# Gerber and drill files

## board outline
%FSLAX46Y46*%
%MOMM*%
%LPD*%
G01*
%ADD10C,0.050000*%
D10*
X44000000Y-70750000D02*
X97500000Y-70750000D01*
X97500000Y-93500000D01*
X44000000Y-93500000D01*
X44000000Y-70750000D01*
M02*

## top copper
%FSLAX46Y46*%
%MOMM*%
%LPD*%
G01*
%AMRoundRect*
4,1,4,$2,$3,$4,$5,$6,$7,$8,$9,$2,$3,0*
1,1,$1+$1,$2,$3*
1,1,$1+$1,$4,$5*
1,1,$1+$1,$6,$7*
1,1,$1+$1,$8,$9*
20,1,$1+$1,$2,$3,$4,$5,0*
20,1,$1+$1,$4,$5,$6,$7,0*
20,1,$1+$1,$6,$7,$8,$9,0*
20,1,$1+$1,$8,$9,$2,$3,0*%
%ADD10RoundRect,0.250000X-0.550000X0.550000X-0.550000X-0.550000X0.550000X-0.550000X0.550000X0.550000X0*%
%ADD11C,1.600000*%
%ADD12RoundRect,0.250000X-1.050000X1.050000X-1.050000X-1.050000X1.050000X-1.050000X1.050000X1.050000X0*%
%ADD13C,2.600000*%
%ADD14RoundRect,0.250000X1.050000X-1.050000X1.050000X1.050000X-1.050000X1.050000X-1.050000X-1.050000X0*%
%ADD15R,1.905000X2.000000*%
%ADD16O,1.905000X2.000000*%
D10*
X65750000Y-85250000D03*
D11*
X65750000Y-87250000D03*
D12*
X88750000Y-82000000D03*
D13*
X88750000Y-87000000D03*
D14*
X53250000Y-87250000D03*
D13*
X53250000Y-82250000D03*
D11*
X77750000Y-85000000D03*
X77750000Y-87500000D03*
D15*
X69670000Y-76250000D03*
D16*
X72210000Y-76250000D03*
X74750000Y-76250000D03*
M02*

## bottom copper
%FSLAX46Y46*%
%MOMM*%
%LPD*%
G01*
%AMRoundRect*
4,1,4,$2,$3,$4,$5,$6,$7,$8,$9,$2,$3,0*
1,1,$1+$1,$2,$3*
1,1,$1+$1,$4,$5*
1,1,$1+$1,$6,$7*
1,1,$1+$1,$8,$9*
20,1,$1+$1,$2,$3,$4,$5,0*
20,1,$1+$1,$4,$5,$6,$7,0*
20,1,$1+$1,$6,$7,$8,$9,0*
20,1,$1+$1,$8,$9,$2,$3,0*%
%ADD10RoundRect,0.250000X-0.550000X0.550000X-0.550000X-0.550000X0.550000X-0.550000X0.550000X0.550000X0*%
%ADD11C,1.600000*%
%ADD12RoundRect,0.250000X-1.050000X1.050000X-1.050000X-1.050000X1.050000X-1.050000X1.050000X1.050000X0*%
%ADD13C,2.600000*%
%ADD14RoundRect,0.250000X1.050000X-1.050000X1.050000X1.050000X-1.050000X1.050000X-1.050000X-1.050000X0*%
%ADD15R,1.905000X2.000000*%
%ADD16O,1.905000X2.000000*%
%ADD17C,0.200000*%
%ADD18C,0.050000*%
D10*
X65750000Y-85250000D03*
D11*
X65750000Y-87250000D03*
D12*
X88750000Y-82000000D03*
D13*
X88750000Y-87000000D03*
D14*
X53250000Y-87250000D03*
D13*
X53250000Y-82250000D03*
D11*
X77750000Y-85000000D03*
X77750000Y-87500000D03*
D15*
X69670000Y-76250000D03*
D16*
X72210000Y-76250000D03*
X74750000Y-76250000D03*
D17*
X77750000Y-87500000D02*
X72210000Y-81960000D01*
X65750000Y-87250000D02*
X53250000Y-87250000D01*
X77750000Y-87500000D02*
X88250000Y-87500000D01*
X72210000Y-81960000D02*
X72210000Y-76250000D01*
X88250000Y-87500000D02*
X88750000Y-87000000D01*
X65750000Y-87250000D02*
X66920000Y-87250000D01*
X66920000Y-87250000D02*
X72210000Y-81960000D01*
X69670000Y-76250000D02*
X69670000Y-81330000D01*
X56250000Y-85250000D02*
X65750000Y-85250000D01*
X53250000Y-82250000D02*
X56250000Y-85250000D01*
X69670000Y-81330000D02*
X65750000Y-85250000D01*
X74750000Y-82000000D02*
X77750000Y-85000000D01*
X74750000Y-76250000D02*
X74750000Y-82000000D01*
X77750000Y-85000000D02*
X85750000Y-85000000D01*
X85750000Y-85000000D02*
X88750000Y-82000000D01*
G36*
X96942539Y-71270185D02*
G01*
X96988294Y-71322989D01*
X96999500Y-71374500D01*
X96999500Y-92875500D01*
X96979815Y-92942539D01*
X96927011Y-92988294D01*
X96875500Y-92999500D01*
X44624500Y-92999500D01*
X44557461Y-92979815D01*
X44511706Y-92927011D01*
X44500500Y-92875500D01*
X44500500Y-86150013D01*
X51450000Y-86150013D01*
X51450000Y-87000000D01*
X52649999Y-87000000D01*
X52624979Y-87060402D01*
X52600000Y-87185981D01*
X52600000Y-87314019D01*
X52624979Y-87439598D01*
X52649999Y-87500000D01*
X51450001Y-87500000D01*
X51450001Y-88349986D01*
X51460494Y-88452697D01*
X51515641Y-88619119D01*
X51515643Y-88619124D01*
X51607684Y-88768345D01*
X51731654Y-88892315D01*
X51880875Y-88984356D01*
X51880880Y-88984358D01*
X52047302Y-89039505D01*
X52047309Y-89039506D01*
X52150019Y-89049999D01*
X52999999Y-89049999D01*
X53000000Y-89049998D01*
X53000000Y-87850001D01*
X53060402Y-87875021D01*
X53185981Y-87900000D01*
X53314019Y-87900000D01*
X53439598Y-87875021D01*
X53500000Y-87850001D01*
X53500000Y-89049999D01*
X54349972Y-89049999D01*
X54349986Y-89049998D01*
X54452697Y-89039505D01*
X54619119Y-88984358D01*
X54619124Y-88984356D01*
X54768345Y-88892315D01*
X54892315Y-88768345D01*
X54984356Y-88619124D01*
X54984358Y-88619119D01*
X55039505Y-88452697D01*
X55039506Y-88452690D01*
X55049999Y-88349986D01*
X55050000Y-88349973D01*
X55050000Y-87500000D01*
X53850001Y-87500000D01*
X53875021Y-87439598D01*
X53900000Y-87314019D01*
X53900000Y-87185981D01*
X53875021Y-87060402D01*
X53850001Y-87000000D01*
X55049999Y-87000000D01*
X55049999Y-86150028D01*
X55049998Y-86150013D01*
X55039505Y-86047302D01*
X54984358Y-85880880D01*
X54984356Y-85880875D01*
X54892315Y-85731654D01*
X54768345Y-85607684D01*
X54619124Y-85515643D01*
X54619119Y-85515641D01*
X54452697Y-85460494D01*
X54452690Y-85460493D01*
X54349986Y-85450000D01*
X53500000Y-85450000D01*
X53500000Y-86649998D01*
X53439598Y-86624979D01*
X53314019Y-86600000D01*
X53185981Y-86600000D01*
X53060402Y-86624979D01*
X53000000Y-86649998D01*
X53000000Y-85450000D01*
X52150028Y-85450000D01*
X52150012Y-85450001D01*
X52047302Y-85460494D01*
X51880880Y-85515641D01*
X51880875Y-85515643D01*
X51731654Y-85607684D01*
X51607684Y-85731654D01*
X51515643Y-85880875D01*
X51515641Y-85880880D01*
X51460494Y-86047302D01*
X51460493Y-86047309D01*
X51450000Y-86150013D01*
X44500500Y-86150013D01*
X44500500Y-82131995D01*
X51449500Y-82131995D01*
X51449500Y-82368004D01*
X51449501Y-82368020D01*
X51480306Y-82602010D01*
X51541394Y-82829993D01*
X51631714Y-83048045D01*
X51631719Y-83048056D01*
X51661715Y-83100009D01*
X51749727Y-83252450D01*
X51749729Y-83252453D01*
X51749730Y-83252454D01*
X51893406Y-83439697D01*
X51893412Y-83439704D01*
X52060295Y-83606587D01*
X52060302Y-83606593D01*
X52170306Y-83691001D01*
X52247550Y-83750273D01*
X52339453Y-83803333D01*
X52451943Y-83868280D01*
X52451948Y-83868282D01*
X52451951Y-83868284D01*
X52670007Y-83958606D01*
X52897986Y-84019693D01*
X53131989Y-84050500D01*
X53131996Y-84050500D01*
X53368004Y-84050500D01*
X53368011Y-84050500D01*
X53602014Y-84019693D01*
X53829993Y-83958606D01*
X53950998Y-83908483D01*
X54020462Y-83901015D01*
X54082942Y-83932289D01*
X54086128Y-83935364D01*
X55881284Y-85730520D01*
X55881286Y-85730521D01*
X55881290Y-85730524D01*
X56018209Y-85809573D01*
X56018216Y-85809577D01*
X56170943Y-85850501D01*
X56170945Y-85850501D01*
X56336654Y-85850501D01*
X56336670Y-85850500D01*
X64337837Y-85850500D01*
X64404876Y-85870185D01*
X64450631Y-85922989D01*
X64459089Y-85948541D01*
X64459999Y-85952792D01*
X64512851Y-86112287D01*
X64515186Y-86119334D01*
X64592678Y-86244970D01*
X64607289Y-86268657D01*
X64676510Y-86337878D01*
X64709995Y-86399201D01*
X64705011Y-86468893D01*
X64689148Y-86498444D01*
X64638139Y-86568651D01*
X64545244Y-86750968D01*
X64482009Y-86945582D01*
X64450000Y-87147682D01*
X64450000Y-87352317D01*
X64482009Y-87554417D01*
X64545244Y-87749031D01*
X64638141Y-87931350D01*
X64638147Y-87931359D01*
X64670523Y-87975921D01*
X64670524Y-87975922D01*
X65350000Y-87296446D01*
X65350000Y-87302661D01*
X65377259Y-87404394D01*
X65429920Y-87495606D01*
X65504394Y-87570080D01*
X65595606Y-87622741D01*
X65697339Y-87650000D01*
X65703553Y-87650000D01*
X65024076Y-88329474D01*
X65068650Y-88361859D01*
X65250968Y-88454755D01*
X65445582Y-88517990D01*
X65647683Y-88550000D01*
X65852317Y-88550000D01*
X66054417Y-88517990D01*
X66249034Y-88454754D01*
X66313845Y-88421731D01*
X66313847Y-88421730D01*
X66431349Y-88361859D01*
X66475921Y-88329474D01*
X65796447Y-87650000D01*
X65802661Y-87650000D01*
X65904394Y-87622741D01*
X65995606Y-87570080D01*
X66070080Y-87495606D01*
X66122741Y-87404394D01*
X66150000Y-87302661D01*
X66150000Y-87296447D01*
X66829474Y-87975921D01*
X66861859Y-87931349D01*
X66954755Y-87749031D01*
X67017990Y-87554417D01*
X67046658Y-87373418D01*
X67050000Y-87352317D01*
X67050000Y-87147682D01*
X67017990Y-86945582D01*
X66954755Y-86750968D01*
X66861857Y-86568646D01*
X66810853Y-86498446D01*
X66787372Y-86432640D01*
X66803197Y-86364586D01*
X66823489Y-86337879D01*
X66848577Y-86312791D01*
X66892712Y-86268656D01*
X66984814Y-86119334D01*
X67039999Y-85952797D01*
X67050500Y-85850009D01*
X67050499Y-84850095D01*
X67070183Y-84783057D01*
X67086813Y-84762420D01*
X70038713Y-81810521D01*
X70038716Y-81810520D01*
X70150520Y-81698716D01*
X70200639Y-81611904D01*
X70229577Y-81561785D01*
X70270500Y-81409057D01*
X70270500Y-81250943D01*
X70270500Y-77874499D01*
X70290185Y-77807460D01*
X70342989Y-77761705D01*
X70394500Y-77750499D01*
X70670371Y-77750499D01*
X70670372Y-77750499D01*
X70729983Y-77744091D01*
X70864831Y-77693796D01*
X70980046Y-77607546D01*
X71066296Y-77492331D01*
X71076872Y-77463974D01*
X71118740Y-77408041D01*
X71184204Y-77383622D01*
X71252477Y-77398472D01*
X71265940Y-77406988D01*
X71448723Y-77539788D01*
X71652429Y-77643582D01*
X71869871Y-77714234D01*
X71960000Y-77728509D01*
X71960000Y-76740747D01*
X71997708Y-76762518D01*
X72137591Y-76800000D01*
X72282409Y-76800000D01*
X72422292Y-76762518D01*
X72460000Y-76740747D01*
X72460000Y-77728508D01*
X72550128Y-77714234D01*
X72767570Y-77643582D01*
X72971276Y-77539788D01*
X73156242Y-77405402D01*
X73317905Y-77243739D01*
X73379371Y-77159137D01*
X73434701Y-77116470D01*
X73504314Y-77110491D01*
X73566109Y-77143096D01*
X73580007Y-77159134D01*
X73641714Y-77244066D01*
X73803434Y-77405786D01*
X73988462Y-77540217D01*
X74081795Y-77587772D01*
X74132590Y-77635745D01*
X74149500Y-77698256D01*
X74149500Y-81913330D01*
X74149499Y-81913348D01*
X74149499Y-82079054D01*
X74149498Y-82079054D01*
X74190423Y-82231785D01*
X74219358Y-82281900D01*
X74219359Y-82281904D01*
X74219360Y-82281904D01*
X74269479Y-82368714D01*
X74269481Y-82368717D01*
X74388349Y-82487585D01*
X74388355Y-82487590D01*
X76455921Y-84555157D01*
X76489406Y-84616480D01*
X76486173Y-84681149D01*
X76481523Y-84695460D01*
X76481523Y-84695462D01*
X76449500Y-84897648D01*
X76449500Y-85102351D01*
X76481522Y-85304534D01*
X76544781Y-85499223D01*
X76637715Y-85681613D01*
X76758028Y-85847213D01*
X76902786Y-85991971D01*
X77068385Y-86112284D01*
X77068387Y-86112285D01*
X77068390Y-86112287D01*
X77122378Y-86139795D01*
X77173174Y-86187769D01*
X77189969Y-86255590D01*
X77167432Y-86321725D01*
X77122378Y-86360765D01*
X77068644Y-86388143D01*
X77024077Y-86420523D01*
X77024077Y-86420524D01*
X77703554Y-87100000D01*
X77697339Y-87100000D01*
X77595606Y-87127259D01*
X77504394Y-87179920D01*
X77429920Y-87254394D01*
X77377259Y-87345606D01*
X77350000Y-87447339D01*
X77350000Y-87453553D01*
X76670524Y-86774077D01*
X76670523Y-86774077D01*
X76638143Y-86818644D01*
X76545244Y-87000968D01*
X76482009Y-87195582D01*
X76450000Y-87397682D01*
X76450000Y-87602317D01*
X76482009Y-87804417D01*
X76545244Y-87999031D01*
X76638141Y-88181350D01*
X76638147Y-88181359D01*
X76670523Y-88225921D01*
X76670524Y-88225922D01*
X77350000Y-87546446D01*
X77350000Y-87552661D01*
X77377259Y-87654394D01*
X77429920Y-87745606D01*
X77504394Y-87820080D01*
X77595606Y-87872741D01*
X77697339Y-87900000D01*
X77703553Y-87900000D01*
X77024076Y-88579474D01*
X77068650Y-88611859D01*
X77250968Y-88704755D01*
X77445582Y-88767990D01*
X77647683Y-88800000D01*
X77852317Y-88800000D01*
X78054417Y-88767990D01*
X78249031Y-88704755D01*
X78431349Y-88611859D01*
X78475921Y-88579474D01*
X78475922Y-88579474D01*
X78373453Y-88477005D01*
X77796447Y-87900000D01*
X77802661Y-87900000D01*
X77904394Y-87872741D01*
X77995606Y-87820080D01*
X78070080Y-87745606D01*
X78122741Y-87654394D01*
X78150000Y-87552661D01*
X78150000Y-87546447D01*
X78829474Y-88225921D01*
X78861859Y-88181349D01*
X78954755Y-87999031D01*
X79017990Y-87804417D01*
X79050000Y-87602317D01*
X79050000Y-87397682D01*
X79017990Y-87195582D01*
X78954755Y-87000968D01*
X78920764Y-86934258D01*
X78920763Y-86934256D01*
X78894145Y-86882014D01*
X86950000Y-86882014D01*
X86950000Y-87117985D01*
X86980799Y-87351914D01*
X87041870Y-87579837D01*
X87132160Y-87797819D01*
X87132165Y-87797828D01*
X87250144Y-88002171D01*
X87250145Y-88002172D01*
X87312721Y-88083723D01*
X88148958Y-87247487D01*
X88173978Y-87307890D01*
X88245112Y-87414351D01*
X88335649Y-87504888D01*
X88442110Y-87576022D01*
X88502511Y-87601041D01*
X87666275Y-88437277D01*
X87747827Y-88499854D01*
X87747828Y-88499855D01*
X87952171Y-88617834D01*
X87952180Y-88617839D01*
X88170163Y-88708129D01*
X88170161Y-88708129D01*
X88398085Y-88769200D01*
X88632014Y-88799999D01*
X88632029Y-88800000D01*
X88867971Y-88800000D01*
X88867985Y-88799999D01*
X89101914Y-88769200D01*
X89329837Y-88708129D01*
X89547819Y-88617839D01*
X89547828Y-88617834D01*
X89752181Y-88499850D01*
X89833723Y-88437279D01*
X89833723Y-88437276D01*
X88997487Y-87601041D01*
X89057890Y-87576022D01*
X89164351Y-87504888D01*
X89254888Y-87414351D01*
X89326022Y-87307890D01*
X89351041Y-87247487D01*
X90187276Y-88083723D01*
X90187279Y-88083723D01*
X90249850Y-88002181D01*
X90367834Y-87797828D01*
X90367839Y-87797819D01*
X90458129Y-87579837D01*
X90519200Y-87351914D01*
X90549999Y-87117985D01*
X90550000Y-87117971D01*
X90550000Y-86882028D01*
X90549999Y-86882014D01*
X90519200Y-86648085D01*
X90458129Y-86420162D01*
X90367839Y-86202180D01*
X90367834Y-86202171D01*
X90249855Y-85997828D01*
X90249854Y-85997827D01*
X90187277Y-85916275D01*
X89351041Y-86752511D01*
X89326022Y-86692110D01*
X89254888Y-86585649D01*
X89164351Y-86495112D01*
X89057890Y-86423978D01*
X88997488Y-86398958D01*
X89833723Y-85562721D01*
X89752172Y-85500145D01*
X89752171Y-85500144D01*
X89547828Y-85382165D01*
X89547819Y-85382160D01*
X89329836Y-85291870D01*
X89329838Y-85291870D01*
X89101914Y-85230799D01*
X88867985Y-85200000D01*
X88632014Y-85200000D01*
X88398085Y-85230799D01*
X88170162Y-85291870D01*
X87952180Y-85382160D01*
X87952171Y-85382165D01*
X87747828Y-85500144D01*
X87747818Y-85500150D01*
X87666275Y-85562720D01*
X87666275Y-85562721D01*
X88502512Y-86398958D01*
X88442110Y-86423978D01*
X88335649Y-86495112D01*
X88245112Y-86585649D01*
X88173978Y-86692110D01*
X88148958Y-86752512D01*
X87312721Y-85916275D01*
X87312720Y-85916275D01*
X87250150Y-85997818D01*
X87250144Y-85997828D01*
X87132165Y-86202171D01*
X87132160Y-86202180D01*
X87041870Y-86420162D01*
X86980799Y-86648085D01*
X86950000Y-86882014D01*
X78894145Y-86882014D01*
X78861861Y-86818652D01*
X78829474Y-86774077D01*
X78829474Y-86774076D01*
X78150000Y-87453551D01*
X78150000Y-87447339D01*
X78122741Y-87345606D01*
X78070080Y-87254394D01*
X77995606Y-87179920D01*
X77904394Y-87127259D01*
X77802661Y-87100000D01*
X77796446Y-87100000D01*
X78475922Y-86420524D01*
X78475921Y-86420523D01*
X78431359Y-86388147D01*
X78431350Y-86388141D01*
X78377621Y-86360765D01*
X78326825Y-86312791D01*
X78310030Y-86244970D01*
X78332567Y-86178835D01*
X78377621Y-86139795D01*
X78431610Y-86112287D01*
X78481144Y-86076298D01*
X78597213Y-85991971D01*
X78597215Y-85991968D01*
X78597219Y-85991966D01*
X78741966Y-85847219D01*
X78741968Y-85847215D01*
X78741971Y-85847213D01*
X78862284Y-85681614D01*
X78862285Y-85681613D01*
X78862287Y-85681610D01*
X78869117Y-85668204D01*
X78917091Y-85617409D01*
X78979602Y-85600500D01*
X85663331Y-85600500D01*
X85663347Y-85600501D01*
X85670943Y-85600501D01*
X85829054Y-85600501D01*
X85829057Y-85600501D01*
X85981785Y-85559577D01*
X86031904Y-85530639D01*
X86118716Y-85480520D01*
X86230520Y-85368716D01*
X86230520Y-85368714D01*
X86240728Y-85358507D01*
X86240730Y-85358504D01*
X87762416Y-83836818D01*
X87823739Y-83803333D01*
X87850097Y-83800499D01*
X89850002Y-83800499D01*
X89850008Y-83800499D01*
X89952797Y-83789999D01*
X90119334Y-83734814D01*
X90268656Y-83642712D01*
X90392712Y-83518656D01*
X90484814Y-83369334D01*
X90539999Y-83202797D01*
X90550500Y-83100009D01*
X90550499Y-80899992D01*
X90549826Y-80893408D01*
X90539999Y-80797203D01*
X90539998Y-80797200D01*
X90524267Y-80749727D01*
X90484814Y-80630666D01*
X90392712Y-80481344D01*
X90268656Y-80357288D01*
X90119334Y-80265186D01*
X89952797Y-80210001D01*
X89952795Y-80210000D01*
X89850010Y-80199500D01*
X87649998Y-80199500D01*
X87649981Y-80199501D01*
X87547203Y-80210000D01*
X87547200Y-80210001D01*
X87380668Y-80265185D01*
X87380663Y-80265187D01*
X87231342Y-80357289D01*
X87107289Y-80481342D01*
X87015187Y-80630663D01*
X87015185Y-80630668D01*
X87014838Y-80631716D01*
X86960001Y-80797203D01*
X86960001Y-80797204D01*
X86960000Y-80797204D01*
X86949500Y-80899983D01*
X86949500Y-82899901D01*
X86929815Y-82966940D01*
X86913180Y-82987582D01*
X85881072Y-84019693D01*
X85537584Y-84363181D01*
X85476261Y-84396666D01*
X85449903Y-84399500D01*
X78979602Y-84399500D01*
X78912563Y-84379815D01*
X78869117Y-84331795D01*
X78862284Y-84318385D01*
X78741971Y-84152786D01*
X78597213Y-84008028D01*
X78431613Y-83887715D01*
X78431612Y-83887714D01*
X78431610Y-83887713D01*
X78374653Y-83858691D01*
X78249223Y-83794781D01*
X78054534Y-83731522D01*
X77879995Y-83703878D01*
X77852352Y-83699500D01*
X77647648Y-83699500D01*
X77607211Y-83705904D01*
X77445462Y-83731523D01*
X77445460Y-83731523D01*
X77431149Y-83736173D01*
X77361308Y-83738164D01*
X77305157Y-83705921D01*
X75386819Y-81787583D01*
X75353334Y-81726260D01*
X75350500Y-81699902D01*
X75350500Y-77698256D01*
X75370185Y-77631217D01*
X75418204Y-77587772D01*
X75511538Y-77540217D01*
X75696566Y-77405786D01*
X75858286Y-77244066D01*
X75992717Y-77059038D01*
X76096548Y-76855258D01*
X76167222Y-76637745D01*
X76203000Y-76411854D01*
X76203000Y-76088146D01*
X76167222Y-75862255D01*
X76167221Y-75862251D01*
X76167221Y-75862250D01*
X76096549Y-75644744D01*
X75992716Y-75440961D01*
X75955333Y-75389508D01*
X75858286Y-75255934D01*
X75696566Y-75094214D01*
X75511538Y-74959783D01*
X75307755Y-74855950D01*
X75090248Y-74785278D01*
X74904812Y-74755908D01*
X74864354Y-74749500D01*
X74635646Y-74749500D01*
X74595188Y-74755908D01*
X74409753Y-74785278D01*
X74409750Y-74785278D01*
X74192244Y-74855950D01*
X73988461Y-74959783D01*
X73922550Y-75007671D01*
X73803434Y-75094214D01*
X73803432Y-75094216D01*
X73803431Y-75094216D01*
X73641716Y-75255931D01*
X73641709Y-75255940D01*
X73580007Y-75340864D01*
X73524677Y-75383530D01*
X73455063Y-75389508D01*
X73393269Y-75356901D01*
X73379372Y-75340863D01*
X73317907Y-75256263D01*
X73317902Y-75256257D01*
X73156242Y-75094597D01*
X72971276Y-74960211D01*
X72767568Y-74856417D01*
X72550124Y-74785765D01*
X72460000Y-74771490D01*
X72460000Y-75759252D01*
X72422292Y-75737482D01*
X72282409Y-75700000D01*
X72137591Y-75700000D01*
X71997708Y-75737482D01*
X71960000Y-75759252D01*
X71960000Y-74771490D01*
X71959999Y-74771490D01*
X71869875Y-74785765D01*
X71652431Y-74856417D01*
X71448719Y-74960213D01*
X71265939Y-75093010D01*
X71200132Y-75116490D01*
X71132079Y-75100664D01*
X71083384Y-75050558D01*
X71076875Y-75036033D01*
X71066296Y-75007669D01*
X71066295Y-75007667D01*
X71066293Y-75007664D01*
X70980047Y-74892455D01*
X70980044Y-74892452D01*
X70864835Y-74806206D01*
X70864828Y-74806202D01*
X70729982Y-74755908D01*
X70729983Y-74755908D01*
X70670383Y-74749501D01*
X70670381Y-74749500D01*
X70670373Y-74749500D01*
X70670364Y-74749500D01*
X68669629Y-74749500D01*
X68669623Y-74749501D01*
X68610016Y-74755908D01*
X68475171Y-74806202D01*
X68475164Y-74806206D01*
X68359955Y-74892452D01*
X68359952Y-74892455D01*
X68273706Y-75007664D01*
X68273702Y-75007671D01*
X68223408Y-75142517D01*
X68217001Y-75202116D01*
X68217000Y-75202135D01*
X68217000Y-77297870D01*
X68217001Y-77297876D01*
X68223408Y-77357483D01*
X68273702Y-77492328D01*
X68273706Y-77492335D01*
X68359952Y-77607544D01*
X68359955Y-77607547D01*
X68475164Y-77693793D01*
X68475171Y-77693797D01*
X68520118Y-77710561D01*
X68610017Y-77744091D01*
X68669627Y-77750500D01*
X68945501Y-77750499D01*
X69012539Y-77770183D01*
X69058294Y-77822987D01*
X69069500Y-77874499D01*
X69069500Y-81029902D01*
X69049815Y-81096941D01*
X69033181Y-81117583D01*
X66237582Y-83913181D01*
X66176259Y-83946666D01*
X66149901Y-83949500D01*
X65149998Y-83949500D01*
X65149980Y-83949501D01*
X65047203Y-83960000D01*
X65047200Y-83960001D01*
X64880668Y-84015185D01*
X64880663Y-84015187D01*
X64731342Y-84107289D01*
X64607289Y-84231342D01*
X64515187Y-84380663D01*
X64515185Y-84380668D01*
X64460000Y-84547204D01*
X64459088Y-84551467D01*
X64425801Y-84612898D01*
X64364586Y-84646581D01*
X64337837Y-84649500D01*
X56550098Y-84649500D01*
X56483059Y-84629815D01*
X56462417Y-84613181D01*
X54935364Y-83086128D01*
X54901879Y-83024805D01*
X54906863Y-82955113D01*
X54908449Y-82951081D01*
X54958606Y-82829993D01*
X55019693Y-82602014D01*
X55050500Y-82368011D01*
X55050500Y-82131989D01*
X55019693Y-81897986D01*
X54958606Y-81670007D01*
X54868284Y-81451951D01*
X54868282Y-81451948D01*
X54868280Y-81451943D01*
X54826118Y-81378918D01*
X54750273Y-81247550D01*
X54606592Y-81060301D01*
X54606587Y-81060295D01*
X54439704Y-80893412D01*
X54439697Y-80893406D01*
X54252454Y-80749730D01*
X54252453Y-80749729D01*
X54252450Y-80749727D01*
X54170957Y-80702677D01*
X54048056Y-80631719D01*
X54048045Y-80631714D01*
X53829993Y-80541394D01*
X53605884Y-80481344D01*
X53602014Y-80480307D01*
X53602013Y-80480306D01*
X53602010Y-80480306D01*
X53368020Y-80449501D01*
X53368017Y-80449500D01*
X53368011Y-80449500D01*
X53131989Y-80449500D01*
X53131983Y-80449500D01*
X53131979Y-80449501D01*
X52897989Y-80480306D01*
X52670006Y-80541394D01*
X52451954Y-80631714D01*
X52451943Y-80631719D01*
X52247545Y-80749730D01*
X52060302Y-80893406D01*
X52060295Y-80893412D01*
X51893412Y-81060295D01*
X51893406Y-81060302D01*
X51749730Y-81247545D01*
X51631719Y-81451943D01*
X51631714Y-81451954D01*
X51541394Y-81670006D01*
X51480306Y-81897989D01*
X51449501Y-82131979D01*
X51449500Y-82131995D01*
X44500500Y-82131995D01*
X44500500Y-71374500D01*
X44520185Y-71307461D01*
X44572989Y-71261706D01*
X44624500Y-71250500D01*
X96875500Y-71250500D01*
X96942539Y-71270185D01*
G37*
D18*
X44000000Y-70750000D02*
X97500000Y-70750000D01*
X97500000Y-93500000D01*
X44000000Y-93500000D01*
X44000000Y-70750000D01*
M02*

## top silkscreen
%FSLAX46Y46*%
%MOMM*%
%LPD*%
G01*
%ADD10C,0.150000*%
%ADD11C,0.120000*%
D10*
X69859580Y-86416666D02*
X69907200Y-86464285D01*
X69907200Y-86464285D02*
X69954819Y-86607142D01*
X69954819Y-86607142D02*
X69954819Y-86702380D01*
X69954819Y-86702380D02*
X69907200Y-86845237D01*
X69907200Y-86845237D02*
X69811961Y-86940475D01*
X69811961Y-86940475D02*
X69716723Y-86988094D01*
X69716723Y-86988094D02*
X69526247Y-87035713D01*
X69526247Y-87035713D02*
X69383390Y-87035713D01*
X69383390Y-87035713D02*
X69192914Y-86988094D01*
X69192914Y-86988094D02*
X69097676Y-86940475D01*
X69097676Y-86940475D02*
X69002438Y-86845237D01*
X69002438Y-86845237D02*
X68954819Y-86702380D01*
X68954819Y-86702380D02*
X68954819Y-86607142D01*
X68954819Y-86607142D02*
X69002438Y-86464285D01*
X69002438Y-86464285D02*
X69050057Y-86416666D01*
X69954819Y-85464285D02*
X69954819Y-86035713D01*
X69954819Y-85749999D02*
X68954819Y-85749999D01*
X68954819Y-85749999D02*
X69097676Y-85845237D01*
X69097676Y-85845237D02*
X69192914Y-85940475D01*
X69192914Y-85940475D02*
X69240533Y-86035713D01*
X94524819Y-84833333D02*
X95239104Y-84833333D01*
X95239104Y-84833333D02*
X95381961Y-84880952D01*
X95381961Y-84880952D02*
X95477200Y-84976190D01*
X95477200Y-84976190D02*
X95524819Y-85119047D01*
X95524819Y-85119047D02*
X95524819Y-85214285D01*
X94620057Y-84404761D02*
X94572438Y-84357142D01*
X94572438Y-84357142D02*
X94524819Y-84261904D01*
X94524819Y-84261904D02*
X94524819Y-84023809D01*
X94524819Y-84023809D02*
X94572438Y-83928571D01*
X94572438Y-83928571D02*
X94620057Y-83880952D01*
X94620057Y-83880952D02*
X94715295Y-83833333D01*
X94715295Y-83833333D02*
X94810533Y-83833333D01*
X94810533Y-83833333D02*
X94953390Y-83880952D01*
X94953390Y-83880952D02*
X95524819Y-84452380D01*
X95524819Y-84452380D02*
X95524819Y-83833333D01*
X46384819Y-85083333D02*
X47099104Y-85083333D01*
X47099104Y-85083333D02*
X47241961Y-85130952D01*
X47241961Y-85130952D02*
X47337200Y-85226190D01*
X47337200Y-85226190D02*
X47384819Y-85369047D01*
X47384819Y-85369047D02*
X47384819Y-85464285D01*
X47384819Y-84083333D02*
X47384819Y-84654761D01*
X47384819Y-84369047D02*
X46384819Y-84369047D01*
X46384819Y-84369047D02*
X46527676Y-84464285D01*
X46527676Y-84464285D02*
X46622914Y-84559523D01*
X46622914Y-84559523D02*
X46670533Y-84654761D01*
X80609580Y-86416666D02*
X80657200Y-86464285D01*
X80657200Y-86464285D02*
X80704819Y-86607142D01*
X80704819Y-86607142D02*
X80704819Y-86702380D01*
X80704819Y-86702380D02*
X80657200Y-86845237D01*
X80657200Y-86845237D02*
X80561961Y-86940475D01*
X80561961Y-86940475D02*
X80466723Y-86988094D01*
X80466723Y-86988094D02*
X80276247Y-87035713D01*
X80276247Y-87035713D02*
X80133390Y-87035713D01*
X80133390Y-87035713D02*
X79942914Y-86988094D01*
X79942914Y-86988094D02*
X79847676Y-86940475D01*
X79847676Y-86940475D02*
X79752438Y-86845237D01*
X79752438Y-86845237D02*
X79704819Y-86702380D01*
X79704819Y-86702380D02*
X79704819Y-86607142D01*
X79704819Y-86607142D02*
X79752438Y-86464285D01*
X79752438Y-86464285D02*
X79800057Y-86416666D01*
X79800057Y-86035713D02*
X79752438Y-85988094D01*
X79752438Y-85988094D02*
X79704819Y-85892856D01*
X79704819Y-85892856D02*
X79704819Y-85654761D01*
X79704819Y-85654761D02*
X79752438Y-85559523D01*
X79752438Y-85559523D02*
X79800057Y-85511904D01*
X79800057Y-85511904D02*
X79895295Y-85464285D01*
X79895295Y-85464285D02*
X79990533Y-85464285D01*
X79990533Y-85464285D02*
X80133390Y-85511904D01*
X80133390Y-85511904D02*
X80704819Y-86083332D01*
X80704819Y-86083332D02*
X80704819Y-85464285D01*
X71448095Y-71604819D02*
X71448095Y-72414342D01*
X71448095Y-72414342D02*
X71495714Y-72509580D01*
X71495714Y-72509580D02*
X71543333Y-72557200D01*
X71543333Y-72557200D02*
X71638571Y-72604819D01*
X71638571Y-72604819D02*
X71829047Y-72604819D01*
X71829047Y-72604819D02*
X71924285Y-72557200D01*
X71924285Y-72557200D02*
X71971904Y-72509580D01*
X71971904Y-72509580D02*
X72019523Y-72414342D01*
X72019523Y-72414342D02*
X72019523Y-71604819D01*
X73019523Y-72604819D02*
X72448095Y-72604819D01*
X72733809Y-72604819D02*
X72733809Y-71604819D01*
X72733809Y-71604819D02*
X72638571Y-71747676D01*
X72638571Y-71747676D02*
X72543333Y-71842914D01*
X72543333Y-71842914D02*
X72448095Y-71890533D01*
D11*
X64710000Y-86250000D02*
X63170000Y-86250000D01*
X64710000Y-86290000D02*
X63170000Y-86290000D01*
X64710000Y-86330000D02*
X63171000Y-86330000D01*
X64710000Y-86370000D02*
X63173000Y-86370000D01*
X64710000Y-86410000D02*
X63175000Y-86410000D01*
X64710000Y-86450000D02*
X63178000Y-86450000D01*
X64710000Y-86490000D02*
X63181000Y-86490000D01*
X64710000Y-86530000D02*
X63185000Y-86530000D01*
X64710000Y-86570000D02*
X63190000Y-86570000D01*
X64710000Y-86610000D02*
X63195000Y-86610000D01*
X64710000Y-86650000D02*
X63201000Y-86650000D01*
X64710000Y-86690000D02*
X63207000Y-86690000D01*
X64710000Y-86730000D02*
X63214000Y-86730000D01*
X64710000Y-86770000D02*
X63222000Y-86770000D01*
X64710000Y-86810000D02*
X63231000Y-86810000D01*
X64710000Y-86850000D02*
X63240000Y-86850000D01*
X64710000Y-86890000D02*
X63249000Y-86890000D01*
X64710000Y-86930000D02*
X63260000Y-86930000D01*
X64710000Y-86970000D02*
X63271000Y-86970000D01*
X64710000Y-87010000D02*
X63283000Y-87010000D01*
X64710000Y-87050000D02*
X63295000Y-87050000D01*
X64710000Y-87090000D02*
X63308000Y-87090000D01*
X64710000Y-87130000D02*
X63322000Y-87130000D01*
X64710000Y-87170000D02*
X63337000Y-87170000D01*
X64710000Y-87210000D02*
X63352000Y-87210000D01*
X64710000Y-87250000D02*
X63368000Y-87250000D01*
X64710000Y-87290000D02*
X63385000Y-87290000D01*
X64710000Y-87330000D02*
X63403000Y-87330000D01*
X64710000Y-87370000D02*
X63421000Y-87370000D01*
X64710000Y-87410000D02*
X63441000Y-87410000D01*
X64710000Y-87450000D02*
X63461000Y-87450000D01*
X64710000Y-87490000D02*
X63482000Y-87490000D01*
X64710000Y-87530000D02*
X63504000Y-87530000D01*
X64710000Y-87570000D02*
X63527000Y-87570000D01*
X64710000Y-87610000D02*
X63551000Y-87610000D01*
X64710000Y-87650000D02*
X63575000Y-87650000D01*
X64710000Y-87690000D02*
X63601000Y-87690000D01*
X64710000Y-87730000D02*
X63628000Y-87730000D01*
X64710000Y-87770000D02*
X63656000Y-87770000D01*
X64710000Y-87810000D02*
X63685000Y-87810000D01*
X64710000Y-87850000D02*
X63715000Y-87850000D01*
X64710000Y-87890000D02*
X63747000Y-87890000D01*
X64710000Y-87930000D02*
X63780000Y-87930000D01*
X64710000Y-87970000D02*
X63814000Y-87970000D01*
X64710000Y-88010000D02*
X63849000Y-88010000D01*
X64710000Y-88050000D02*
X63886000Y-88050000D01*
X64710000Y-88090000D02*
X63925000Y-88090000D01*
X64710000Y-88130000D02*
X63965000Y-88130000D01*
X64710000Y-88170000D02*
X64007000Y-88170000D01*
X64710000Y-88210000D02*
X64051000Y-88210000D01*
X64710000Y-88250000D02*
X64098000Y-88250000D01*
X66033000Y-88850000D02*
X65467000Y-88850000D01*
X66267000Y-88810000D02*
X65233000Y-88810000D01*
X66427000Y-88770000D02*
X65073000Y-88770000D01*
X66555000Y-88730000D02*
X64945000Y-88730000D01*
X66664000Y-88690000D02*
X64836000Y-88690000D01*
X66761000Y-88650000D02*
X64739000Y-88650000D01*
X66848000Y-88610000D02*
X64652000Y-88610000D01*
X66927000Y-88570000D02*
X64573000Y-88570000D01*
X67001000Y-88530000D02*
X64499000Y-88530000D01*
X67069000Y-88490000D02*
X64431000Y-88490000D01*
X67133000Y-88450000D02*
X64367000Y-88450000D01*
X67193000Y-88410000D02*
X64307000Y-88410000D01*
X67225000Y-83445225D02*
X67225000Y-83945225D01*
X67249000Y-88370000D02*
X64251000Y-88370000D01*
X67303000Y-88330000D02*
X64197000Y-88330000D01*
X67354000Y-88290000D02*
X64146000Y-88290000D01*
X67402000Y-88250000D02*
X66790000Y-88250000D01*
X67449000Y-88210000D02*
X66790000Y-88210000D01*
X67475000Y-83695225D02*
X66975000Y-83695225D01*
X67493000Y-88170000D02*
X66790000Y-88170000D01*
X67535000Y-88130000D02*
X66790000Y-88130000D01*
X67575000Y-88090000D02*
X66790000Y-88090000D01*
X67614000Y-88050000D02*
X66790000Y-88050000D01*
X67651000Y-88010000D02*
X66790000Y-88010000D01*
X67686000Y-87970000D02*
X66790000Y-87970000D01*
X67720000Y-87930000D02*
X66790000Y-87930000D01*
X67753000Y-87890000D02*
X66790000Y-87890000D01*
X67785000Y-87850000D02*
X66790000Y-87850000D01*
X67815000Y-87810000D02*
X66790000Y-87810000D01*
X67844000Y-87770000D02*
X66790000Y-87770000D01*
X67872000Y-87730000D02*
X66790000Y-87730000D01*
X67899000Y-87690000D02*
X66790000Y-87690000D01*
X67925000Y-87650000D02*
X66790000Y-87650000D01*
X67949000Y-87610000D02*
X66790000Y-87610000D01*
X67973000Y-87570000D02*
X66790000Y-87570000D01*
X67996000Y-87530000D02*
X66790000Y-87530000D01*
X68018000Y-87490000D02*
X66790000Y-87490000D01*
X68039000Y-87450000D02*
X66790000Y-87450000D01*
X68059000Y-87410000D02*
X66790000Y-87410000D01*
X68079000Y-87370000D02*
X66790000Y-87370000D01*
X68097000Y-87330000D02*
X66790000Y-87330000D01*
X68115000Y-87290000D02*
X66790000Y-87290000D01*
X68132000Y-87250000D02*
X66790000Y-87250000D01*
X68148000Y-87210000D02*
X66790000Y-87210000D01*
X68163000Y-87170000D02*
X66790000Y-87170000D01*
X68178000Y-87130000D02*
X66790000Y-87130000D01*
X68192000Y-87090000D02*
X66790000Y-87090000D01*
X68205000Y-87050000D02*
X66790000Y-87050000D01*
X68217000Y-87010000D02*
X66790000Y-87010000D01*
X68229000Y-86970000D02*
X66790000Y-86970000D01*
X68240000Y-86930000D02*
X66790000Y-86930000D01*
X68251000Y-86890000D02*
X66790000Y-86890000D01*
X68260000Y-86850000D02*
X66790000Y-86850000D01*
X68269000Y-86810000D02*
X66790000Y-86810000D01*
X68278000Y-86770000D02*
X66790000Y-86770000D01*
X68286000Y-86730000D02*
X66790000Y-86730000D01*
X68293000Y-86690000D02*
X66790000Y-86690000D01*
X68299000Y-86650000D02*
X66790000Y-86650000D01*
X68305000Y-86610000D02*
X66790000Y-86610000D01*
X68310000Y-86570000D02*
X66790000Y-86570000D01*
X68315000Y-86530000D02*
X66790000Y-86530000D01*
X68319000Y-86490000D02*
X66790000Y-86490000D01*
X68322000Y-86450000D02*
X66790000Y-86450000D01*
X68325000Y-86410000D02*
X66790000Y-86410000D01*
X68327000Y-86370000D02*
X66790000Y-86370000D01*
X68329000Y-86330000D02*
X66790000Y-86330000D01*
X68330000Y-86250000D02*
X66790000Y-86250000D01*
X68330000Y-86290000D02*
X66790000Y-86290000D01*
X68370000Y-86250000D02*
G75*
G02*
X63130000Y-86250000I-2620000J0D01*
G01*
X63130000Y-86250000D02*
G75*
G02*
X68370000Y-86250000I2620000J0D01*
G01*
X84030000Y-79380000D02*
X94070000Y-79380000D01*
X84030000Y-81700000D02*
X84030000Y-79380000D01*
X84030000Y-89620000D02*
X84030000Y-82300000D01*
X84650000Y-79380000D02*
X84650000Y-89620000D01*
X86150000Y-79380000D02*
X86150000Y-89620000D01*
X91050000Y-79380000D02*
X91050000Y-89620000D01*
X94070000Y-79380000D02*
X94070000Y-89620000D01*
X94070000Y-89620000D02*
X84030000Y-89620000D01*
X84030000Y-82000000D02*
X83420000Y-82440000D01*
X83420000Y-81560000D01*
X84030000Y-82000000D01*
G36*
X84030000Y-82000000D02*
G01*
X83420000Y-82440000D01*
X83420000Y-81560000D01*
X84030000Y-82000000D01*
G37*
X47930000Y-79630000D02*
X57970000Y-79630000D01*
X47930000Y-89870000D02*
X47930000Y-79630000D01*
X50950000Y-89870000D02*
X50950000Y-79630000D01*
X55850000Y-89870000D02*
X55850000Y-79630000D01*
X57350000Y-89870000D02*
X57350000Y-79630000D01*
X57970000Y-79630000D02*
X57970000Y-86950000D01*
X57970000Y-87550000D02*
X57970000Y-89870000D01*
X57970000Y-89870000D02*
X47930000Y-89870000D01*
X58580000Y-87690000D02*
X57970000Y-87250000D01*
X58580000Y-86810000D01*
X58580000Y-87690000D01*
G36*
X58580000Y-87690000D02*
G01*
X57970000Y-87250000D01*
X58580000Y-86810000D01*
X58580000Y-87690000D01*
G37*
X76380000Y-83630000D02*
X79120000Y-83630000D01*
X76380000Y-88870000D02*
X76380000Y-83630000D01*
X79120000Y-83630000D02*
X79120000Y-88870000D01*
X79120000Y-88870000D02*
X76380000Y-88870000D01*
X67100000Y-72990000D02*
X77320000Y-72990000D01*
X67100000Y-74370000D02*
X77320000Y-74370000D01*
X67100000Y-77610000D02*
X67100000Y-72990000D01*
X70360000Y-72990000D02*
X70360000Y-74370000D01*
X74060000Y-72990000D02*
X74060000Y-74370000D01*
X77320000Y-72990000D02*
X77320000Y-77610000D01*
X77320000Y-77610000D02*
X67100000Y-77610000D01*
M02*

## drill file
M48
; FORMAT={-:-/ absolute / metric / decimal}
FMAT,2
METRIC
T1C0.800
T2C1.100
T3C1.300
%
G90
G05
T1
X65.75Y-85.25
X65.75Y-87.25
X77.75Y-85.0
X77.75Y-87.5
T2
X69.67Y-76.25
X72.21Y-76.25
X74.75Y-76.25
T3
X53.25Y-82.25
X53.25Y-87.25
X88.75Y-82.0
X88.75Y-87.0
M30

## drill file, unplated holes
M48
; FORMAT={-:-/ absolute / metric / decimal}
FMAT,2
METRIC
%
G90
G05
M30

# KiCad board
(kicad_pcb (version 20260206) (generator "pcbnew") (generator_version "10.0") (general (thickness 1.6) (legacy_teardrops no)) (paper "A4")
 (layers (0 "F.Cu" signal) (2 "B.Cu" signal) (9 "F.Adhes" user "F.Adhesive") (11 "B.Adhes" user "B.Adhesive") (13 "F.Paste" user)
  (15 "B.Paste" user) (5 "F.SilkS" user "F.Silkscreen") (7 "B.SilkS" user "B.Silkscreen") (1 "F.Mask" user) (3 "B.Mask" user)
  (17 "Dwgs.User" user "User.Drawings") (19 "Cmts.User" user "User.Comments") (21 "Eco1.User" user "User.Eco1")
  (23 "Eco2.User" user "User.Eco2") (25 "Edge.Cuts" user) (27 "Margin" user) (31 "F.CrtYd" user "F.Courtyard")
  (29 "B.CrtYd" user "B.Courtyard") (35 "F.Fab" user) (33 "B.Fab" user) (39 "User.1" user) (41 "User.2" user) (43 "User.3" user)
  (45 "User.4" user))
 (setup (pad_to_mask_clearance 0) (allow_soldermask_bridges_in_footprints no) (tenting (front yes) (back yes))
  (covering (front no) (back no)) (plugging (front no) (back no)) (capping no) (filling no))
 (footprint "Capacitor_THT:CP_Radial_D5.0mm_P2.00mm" (layer "F.Cu") (at 65.75 85.25 -90)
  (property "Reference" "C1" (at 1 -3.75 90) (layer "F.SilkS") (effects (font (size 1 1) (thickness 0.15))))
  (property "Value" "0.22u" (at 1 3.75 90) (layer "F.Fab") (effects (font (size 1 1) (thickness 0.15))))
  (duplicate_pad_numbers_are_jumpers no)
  (fp_line (start 1 1.04) (end 1 2.58) (stroke (width 0.12) (type solid)) (layer "F.SilkS"))
  (fp_line (start 1.04 1.04) (end 1.04 2.58) (stroke (width 0.12) (type solid)) (layer "F.SilkS"))
  (fp_line (start 1.08 1.04) (end 1.08 2.579) (stroke (width 0.12) (type solid)) (layer "F.SilkS"))
  (fp_line (start 1.12 1.04) (end 1.12 2.577) (stroke (width 0.12) (type solid)) (layer "F.SilkS"))
  (fp_line (start 1.16 1.04) (end 1.16 2.575) (stroke (width 0.12) (type solid)) (layer "F.SilkS"))
  (fp_line (start 1.2 1.04) (end 1.2 2.572) (stroke (width 0.12) (type solid)) (layer "F.SilkS"))
  (fp_line (start 1.24 1.04) (end 1.24 2.569) (stroke (width 0.12) (type solid)) (layer "F.SilkS"))
  (fp_line (start 1.28 1.04) (end 1.28 2.565) (stroke (width 0.12) (type solid)) (layer "F.SilkS"))
  (fp_line (start 1.32 1.04) (end 1.32 2.56) (stroke (width 0.12) (type solid)) (layer "F.SilkS"))
  (fp_line (start 1.36 1.04) (end 1.36 2.555) (stroke (width 0.12) (type solid)) (layer "F.SilkS"))
  (fp_line (start 1.4 1.04) (end 1.4 2.549) (stroke (width 0.12) (type solid)) (layer "F.SilkS"))
  (fp_line (start 1.44 1.04) (end 1.44 2.543) (stroke (width 0.12) (type solid)) (layer "F.SilkS"))
  (fp_line (start 1.48 1.04) (end 1.48 2.536) (stroke (width 0.12) (type solid)) (layer "F.SilkS"))
  (fp_line (start 1.52 1.04) (end 1.52 2.528) (stroke (width 0.12) (type solid)) (layer "F.SilkS"))
  (fp_line (start 1.56 1.04) (end 1.56 2.519) (stroke (width 0.12) (type solid)) (layer "F.SilkS"))
  (fp_line (start 1.6 1.04) (end 1.6 2.51) (stroke (width 0.12) (type solid)) (layer "F.SilkS"))
  (fp_line (start 1.64 1.04) (end 1.64 2.501) (stroke (width 0.12) (type solid)) (layer "F.SilkS"))
  (fp_line (start 1.68 1.04) (end 1.68 2.49) (stroke (width 0.12) (type solid)) (layer "F.SilkS"))
  (fp_line (start 1.72 1.04) (end 1.72 2.479) (stroke (width 0.12) (type solid)) (layer "F.SilkS"))
  (fp_line (start 1.76 1.04) (end 1.76 2.467) (stroke (width 0.12) (type solid)) (layer "F.SilkS"))
  (fp_line (start 1.8 1.04) (end 1.8 2.455) (stroke (width 0.12) (type solid)) (layer "F.SilkS"))
  (fp_line (start 1.84 1.04) (end 1.84 2.442) (stroke (width 0.12) (type solid)) (layer "F.SilkS"))
  (fp_line (start 1.88 1.04) (end 1.88 2.428) (stroke (width 0.12) (type solid)) (layer "F.SilkS"))
  (fp_line (start 1.92 1.04) (end 1.92 2.413) (stroke (width 0.12) (type solid)) (layer "F.SilkS"))
  (fp_line (start 1.96 1.04) (end 1.96 2.398) (stroke (width 0.12) (type solid)) (layer "F.SilkS"))
  (fp_line (start 2 1.04) (end 2 2.382) (stroke (width 0.12) (type solid)) (layer "F.SilkS"))
  (fp_line (start 2.04 1.04) (end 2.04 2.365) (stroke (width 0.12) (type solid)) (layer "F.SilkS"))
  (fp_line (start 2.08 1.04) (end 2.08 2.347) (stroke (width 0.12) (type solid)) (layer "F.SilkS"))
  (fp_line (start 2.12 1.04) (end 2.12 2.329) (stroke (width 0.12) (type solid)) (layer "F.SilkS"))
  (fp_line (start 2.16 1.04) (end 2.16 2.309) (stroke (width 0.12) (type solid)) (layer "F.SilkS"))
  (fp_line (start 2.2 1.04) (end 2.2 2.289) (stroke (width 0.12) (type solid)) (layer "F.SilkS"))
  (fp_line (start 2.24 1.04) (end 2.24 2.268) (stroke (width 0.12) (type solid)) (layer "F.SilkS"))
  (fp_line (start 2.28 1.04) (end 2.28 2.246) (stroke (width 0.12) (type solid)) (layer "F.SilkS"))
  (fp_line (start 2.32 1.04) (end 2.32 2.223) (stroke (width 0.12) (type solid)) (layer "F.SilkS"))
  (fp_line (start 2.36 1.04) (end 2.36 2.199) (stroke (width 0.12) (type solid)) (layer "F.SilkS"))
  (fp_line (start 2.4 1.04) (end 2.4 2.175) (stroke (width 0.12) (type solid)) (layer "F.SilkS"))
  (fp_line (start 2.44 1.04) (end 2.44 2.149) (stroke (width 0.12) (type solid)) (layer "F.SilkS"))
  (fp_line (start 2.48 1.04) (end 2.48 2.122) (stroke (width 0.12) (type solid)) (layer "F.SilkS"))
  (fp_line (start 2.52 1.04) (end 2.52 2.094) (stroke (width 0.12) (type solid)) (layer "F.SilkS"))
  (fp_line (start 2.56 1.04) (end 2.56 2.065) (stroke (width 0.12) (type solid)) (layer "F.SilkS"))
  (fp_line (start 2.6 1.04) (end 2.6 2.035) (stroke (width 0.12) (type solid)) (layer "F.SilkS"))
  (fp_line (start 2.64 1.04) (end 2.64 2.003) (stroke (width 0.12) (type solid)) (layer "F.SilkS"))
  (fp_line (start 2.68 1.04) (end 2.68 1.97) (stroke (width 0.12) (type solid)) (layer "F.SilkS"))
  (fp_line (start 2.72 1.04) (end 2.72 1.936) (stroke (width 0.12) (type solid)) (layer "F.SilkS"))
  (fp_line (start 2.76 1.04) (end 2.76 1.901) (stroke (width 0.12) (type solid)) (layer "F.SilkS"))
  (fp_line (start 2.8 1.04) (end 2.8 1.864) (stroke (width 0.12) (type solid)) (layer "F.SilkS"))
  (fp_line (start 2.84 1.04) (end 2.84 1.825) (stroke (width 0.12) (type solid)) (layer "F.SilkS"))
  (fp_line (start 2.88 1.04) (end 2.88 1.785) (stroke (width 0.12) (type solid)) (layer "F.SilkS"))
  (fp_line (start 2.92 1.04) (end 2.92 1.743) (stroke (width 0.12) (type solid)) (layer "F.SilkS"))
  (fp_line (start 2.96 1.04) (end 2.96 1.699) (stroke (width 0.12) (type solid)) (layer "F.SilkS"))
  (fp_line (start 3 1.04) (end 3 1.652) (stroke (width 0.12) (type solid)) (layer "F.SilkS"))
  (fp_line (start 3.6 -0.283) (end 3.6 0.283) (stroke (width 0.12) (type solid)) (layer "F.SilkS"))
  (fp_line (start 3.56 -0.517) (end 3.56 0.517) (stroke (width 0.12) (type solid)) (layer "F.SilkS"))
  (fp_line (start 3.52 -0.677) (end 3.52 0.677) (stroke (width 0.12) (type solid)) (layer "F.SilkS"))
  (fp_line (start 3.48 -0.805) (end 3.48 0.805) (stroke (width 0.12) (type solid)) (layer "F.SilkS"))
  (fp_line (start 3.44 -0.914) (end 3.44 0.914) (stroke (width 0.12) (type solid)) (layer "F.SilkS"))
  (fp_line (start 3.4 -1.011) (end 3.4 1.011) (stroke (width 0.12) (type solid)) (layer "F.SilkS"))
  (fp_line (start 3.36 -1.098) (end 3.36 1.098) (stroke (width 0.12) (type solid)) (layer "F.SilkS"))
  (fp_line (start 3.32 -1.177) (end 3.32 1.177) (stroke (width 0.12) (type solid)) (layer "F.SilkS"))
  (fp_line (start 3.28 -1.251) (end 3.28 1.251) (stroke (width 0.12) (type solid)) (layer "F.SilkS"))
  (fp_line (start 3.24 -1.319) (end 3.24 1.319) (stroke (width 0.12) (type solid)) (layer "F.SilkS"))
  (fp_line (start 3.2 -1.383) (end 3.2 1.383) (stroke (width 0.12) (type solid)) (layer "F.SilkS"))
  (fp_line (start 3.16 -1.443) (end 3.16 1.443) (stroke (width 0.12) (type solid)) (layer "F.SilkS"))
  (fp_line (start -1.804775 -1.475) (end -1.304775 -1.475) (stroke (width 0.12) (type solid)) (layer "F.SilkS"))
  (fp_line (start 3.12 -1.499) (end 3.12 1.499) (stroke (width 0.12) (type solid)) (layer "F.SilkS"))
  (fp_line (start 3.08 -1.553) (end 3.08 1.553) (stroke (width 0.12) (type solid)) (layer "F.SilkS"))
  (fp_line (start 3.04 -1.604) (end 3.04 1.604) (stroke (width 0.12) (type solid)) (layer "F.SilkS"))
  (fp_line (start 3 -1.652) (end 3 -1.04) (stroke (width 0.12) (type solid)) (layer "F.SilkS"))
  (fp_line (start 2.96 -1.699) (end 2.96 -1.04) (stroke (width 0.12) (type solid)) (layer "F.SilkS"))
  (fp_line (start -1.554775 -1.725) (end -1.554775 -1.225) (stroke (width 0.12) (type solid)) (layer "F.SilkS"))
  (fp_line (start 2.92 -1.743) (end 2.92 -1.04) (stroke (width 0.12) (type solid)) (layer "F.SilkS"))
  (fp_line (start 2.88 -1.785) (end 2.88 -1.04) (stroke (width 0.12) (type solid)) (layer "F.SilkS"))
  (fp_line (start 2.84 -1.825) (end 2.84 -1.04) (stroke (width 0.12) (type solid)) (layer "F.SilkS"))
  (fp_line (start 2.8 -1.864) (end 2.8 -1.04) (stroke (width 0.12) (type solid)) (layer "F.SilkS"))
  (fp_line (start 2.76 -1.901) (end 2.76 -1.04) (stroke (width 0.12) (type solid)) (layer "F.SilkS"))
  (fp_line (start 2.72 -1.936) (end 2.72 -1.04) (stroke (width 0.12) (type solid)) (layer "F.SilkS"))
  (fp_line (start 2.68 -1.97) (end 2.68 -1.04) (stroke (width 0.12) (type solid)) (layer "F.SilkS"))
  (fp_line (start 2.64 -2.003) (end 2.64 -1.04) (stroke (width 0.12) (type solid)) (layer "F.SilkS"))
  (fp_line (start 2.6 -2.035) (end 2.6 -1.04) (stroke (width 0.12) (type solid)) (layer "F.SilkS"))
  (fp_line (start 2.56 -2.065) (end 2.56 -1.04) (stroke (width 0.12) (type solid)) (layer "F.SilkS"))
  (fp_line (start 2.52 -2.094) (end 2.52 -1.04) (stroke (width 0.12) (type solid)) (layer "F.SilkS"))
  (fp_line (start 2.48 -2.122) (end 2.48 -1.04) (stroke (width 0.12) (type solid)) (layer "F.SilkS"))
  (fp_line (start 2.44 -2.149) (end 2.44 -1.04) (stroke (width 0.12) (type solid)) (layer "F.SilkS"))
  (fp_line (start 2.4 -2.175) (end 2.4 -1.04) (stroke (width 0.12) (type solid)) (layer "F.SilkS"))
  (fp_line (start 2.36 -2.199) (end 2.36 -1.04) (stroke (width 0.12) (type solid)) (layer "F.SilkS"))
  (fp_line (start 2.32 -2.223) (end 2.32 -1.04) (stroke (width 0.12) (type solid)) (layer "F.SilkS"))
  (fp_line (start 2.28 -2.246) (end 2.28 -1.04) (stroke (width 0.12) (type solid)) (layer "F.SilkS"))
  (fp_line (start 2.24 -2.268) (end 2.24 -1.04) (stroke (width 0.12) (type solid)) (layer "F.SilkS"))
  (fp_line (start 2.2 -2.289) (end 2.2 -1.04) (stroke (width 0.12) (type solid)) (layer "F.SilkS"))
  (fp_line (start 2.16 -2.309) (end 2.16 -1.04) (stroke (width 0.12) (type solid)) (layer "F.SilkS"))
  (fp_line (start 2.12 -2.329) (end 2.12 -1.04) (stroke (width 0.12) (type solid)) (layer "F.SilkS"))
  (fp_line (start 2.08 -2.347) (end 2.08 -1.04) (stroke (width 0.12) (type solid)) (layer "F.SilkS"))
  (fp_line (start 2.04 -2.365) (end 2.04 -1.04) (stroke (width 0.12) (type solid)) (layer "F.SilkS"))
  (fp_line (start 2 -2.382) (end 2 -1.04) (stroke (width 0.12) (type solid)) (layer "F.SilkS"))
  (fp_line (start 1.96 -2.398) (end 1.96 -1.04) (stroke (width 0.12) (type solid)) (layer "F.SilkS"))
  (fp_line (start 1.92 -2.413) (end 1.92 -1.04) (stroke (width 0.12) (type solid)) (layer "F.SilkS"))
  (fp_line (start 1.88 -2.428) (end 1.88 -1.04) (stroke (width 0.12) (type solid)) (layer "F.SilkS"))
  (fp_line (start 1.84 -2.442) (end 1.84 -1.04) (stroke (width 0.12) (type solid)) (layer "F.SilkS"))
  (fp_line (start 1.8 -2.455) (end 1.8 -1.04) (stroke (width 0.12) (type solid)) (layer "F.SilkS"))
  (fp_line (start 1.76 -2.467) (end 1.76 -1.04) (stroke (width 0.12) (type solid)) (layer "F.SilkS"))
  (fp_line (start 1.72 -2.479) (end 1.72 -1.04) (stroke (width 0.12) (type solid)) (layer "F.SilkS"))
  (fp_line (start 1.68 -2.49) (end 1.68 -1.04) (stroke (width 0.12) (type solid)) (layer "F.SilkS"))
  (fp_line (start 1.64 -2.501) (end 1.64 -1.04) (stroke (width 0.12) (type solid)) (layer "F.SilkS"))
  (fp_line (start 1.6 -2.51) (end 1.6 -1.04) (stroke (width 0.12) (type solid)) (layer "F.SilkS"))
  (fp_line (start 1.56 -2.519) (end 1.56 -1.04) (stroke (width 0.12) (type solid)) (layer "F.SilkS"))
  (fp_line (start 1.52 -2.528) (end 1.52 -1.04) (stroke (width 0.12) (type solid)) (layer "F.SilkS"))
  (fp_line (start 1.48 -2.536) (end 1.48 -1.04) (stroke (width 0.12) (type solid)) (layer "F.SilkS"))
  (fp_line (start 1.44 -2.543) (end 1.44 -1.04) (stroke (width 0.12) (type solid)) (layer "F.SilkS"))
  (fp_line (start 1.4 -2.549) (end 1.4 -1.04) (stroke (width 0.12) (type solid)) (layer "F.SilkS"))
  (fp_line (start 1.36 -2.555) (end 1.36 -1.04) (stroke (width 0.12) (type solid)) (layer "F.SilkS"))
  (fp_line (start 1.32 -2.56) (end 1.32 -1.04) (stroke (width 0.12) (type solid)) (layer "F.SilkS"))
  (fp_line (start 1.28 -2.565) (end 1.28 -1.04) (stroke (width 0.12) (type solid)) (layer "F.SilkS"))
  (fp_line (start 1.24 -2.569) (end 1.24 -1.04) (stroke (width 0.12) (type solid)) (layer "F.SilkS"))
  (fp_line (start 1.2 -2.572) (end 1.2 -1.04) (stroke (width 0.12) (type solid)) (layer "F.SilkS"))
  (fp_line (start 1.16 -2.575) (end 1.16 -1.04) (stroke (width 0.12) (type solid)) (layer "F.SilkS"))
  (fp_line (start 1.12 -2.577) (end 1.12 -1.04) (stroke (width 0.12) (type solid)) (layer "F.SilkS"))
  (fp_line (start 1.08 -2.579) (end 1.08 -1.04) (stroke (width 0.12) (type solid)) (layer "F.SilkS"))
  (fp_line (start 1 -2.58) (end 1 -1.04) (stroke (width 0.12) (type solid)) (layer "F.SilkS"))
  (fp_line (start 1.04 -2.58) (end 1.04 -1.04) (stroke (width 0.12) (type solid)) (layer "F.SilkS"))
  (fp_circle (center 1 0) (end 3.62 0) (stroke (width 0.12) (type solid)) (fill no) (layer "F.SilkS"))
  (pad "1" thru_hole roundrect (at 0 0 270) (size 1.6 1.6) (drill 0.8) (layers "*.Cu" "*.Mask") (remove_unused_layers no)
   (roundrect_rratio 0.15625) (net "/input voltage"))
  (pad "2" thru_hole circle (at 2 0 270) (size 1.6 1.6) (drill 0.8) (layers "*.Cu" "*.Mask") (remove_unused_layers no) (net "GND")))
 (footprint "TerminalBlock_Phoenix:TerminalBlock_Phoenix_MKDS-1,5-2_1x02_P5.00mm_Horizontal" (layer "F.Cu") (at 88.75 82 -90)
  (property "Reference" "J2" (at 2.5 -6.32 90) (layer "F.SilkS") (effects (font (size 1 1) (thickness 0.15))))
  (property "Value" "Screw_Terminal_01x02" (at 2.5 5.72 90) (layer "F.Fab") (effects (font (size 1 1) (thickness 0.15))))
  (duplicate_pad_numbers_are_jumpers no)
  (fp_line (start -2.62 4.72) (end -2.62 -5.32) (stroke (width 0.12) (type solid)) (layer "F.SilkS"))
  (fp_line (start -0.3 4.72) (end -2.62 4.72) (stroke (width 0.12) (type solid)) (layer "F.SilkS"))
  (fp_line (start 7.62 4.72) (end 0.3 4.72) (stroke (width 0.12) (type solid)) (layer "F.SilkS"))
  (fp_line (start -2.62 4.1) (end 7.62 4.1) (stroke (width 0.12) (type solid)) (layer "F.SilkS"))
  (fp_line (start -2.62 2.6) (end 7.62 2.6) (stroke (width 0.12) (type solid)) (layer "F.SilkS"))
  (fp_line (start -2.62 -2.3) (end 7.62 -2.3) (stroke (width 0.12) (type solid)) (layer "F.SilkS"))
  (fp_line (start -2.62 -5.32) (end 7.62 -5.32) (stroke (width 0.12) (type solid)) (layer "F.SilkS"))
  (fp_line (start 7.62 -5.32) (end 7.62 4.72) (stroke (width 0.12) (type solid)) (layer "F.SilkS"))
  (fp_poly (pts (xy 0 4.72) (xy 0.44 5.33) (xy -0.44 5.33)) (stroke (width 0.12) (type solid)) (fill yes) (layer "F.SilkS"))
  (pad "1" thru_hole roundrect (at 0 0 270) (size 2.6 2.6) (drill 1.3) (layers "*.Cu" "*.Mask") (remove_unused_layers no)
   (roundrect_rratio 0.096154) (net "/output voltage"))
  (pad "2" thru_hole circle (at 5 0 270) (size 2.6 2.6) (drill 1.3) (layers "*.Cu" "*.Mask") (remove_unused_layers no) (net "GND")))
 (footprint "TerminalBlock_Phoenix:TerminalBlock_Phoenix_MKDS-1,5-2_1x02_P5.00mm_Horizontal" (layer "F.Cu") (at 53.25 87.25 90)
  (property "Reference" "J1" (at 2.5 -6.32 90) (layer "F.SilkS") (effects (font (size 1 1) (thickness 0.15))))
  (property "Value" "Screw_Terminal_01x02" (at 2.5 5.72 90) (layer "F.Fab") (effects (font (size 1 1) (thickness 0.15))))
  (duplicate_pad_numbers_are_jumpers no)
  (fp_line (start 7.62 -5.32) (end 7.62 4.72) (stroke (width 0.12) (type solid)) (layer "F.SilkS"))
  (fp_line (start -2.62 -5.32) (end 7.62 -5.32) (stroke (width 0.12) (type solid)) (layer "F.SilkS"))
  (fp_line (start -2.62 -2.3) (end 7.62 -2.3) (stroke (width 0.12) (type solid)) (layer "F.SilkS"))
  (fp_line (start -2.62 2.6) (end 7.62 2.6) (stroke (width 0.12) (type solid)) (layer "F.SilkS"))
  (fp_line (start -2.62 4.1) (end 7.62 4.1) (stroke (width 0.12) (type solid)) (layer "F.SilkS"))
  (fp_line (start 7.62 4.72) (end 0.3 4.72) (stroke (width 0.12) (type solid)) (layer "F.SilkS"))
  (fp_line (start -0.3 4.72) (end -2.62 4.72) (stroke (width 0.12) (type solid)) (layer "F.SilkS"))
  (fp_line (start -2.62 4.72) (end -2.62 -5.32) (stroke (width 0.12) (type solid)) (layer "F.SilkS"))
  (fp_poly (pts (xy 0 4.72) (xy 0.44 5.33) (xy -0.44 5.33)) (stroke (width 0.12) (type solid)) (fill yes) (layer "F.SilkS"))
  (pad "1" thru_hole roundrect (at 0 0 90) (size 2.6 2.6) (drill 1.3) (layers "*.Cu" "*.Mask") (remove_unused_layers no)
   (roundrect_rratio 0.096154) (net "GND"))
  (pad "2" thru_hole circle (at 5 0 90) (size 2.6 2.6) (drill 1.3) (layers "*.Cu" "*.Mask") (remove_unused_layers no) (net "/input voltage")))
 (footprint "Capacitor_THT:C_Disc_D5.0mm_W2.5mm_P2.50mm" (layer "F.Cu") (at 77.75 85 -90)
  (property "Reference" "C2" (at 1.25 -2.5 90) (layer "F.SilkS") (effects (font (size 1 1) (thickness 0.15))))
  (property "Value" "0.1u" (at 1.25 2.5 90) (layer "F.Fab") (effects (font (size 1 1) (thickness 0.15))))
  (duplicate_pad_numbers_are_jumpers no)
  (fp_line (start -1.37 1.37) (end -1.37 -1.37) (stroke (width 0.12) (type solid)) (layer "F.SilkS"))
  (fp_line (start 3.87 1.37) (end -1.37 1.37) (stroke (width 0.12) (type solid)) (layer "F.SilkS"))
  (fp_line (start -1.37 -1.37) (end 3.87 -1.37) (stroke (width 0.12) (type solid)) (layer "F.SilkS"))
  (fp_line (start 3.87 -1.37) (end 3.87 1.37) (stroke (width 0.12) (type solid)) (layer "F.SilkS"))
  (pad "1" thru_hole circle (at 0 0 270) (size 1.6 1.6) (drill 0.8) (layers "*.Cu" "*.Mask") (remove_unused_layers no)
   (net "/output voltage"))
  (pad "2" thru_hole circle (at 2.5 0 270) (size 1.6 1.6) (drill 0.8) (layers "*.Cu" "*.Mask") (remove_unused_layers no) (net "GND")))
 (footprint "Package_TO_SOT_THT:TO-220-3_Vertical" (layer "F.Cu") (at 69.67 76.25)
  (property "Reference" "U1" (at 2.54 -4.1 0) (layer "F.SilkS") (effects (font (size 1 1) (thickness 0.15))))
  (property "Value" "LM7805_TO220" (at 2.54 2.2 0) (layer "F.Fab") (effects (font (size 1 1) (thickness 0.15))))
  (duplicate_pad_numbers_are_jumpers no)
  (fp_line (start -2.57 -3.26) (end 7.65 -3.26) (stroke (width 0.12) (type solid)) (layer "F.SilkS"))
  (fp_line (start -2.57 -1.88) (end 7.65 -1.88) (stroke (width 0.12) (type solid)) (layer "F.SilkS"))
  (fp_line (start -2.57 1.36) (end -2.57 -3.26) (stroke (width 0.12) (type solid)) (layer "F.SilkS"))
  (fp_line (start 0.69 -3.26) (end 0.69 -1.88) (stroke (width 0.12) (type solid)) (layer "F.SilkS"))
  (fp_line (start 4.39 -3.26) (end 4.39 -1.88) (stroke (width 0.12) (type solid)) (layer "F.SilkS"))
  (fp_line (start 7.65 -3.26) (end 7.65 1.36) (stroke (width 0.12) (type solid)) (layer "F.SilkS"))
  (fp_line (start 7.65 1.36) (end -2.57 1.36) (stroke (width 0.12) (type solid)) (layer "F.SilkS"))
  (pad "1" thru_hole rect (at 0 0) (size 1.905 2) (drill 1.1) (layers "*.Cu" "*.Mask") (remove_unused_layers no) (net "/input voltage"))
  (pad "2" thru_hole oval (at 2.54 0) (size 1.905 2) (drill 1.1) (layers "*.Cu" "*.Mask") (remove_unused_layers no) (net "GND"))
  (pad "3" thru_hole oval (at 5.08 0) (size 1.905 2) (drill 1.1) (layers "*.Cu" "*.Mask") (remove_unused_layers no) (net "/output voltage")))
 (gr_rect (start 44 70.75) (end 97.5 93.5) (stroke (width 0.05) (type default)) (fill no) (layer "Edge.Cuts"))
 (segment (start 77.75 87.5) (end 72.21 81.96) (width 0.2) (layer "B.Cu") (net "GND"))
 (segment (start 65.75 87.25) (end 53.25 87.25) (width 0.2) (layer "B.Cu") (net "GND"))
 (segment (start 77.75 87.5) (end 88.25 87.5) (width 0.2) (layer "B.Cu") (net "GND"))
 (segment (start 72.21 81.96) (end 72.21 76.25) (width 0.2) (layer "B.Cu") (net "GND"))
 (segment (start 88.25 87.5) (end 88.75 87) (width 0.2) (layer "B.Cu") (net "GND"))
 (segment (start 65.75 87.25) (end 66.92 87.25) (width 0.2) (layer "B.Cu") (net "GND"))
 (segment (start 66.92 87.25) (end 72.21 81.96) (width 0.2) (layer "B.Cu") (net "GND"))
 (segment (start 69.67 76.25) (end 69.67 81.33) (width 0.2) (layer "B.Cu") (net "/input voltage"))
 (segment (start 56.25 85.25) (end 65.75 85.25) (width 0.2) (layer "B.Cu") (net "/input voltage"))
 (segment (start 53.25 82.25) (end 56.25 85.25) (width 0.2) (layer "B.Cu") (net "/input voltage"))
 (segment (start 69.67 81.33) (end 65.75 85.25) (width 0.2) (layer "B.Cu") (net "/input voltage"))
 (segment (start 74.75 82) (end 77.75 85) (width 0.2) (layer "B.Cu") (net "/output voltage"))
 (segment (start 74.75 76.25) (end 74.75 82) (width 0.2) (layer "B.Cu") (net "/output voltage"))
 (segment (start 77.75 85) (end 85.75 85) (width 0.2) (layer "B.Cu") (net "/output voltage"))
 (segment (start 85.75 85) (end 88.75 82) (width 0.2) (layer "B.Cu") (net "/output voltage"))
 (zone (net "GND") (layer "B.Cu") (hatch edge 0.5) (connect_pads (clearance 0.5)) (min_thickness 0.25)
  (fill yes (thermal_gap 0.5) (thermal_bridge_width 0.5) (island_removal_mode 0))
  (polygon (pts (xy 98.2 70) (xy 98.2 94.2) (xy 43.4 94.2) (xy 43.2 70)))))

